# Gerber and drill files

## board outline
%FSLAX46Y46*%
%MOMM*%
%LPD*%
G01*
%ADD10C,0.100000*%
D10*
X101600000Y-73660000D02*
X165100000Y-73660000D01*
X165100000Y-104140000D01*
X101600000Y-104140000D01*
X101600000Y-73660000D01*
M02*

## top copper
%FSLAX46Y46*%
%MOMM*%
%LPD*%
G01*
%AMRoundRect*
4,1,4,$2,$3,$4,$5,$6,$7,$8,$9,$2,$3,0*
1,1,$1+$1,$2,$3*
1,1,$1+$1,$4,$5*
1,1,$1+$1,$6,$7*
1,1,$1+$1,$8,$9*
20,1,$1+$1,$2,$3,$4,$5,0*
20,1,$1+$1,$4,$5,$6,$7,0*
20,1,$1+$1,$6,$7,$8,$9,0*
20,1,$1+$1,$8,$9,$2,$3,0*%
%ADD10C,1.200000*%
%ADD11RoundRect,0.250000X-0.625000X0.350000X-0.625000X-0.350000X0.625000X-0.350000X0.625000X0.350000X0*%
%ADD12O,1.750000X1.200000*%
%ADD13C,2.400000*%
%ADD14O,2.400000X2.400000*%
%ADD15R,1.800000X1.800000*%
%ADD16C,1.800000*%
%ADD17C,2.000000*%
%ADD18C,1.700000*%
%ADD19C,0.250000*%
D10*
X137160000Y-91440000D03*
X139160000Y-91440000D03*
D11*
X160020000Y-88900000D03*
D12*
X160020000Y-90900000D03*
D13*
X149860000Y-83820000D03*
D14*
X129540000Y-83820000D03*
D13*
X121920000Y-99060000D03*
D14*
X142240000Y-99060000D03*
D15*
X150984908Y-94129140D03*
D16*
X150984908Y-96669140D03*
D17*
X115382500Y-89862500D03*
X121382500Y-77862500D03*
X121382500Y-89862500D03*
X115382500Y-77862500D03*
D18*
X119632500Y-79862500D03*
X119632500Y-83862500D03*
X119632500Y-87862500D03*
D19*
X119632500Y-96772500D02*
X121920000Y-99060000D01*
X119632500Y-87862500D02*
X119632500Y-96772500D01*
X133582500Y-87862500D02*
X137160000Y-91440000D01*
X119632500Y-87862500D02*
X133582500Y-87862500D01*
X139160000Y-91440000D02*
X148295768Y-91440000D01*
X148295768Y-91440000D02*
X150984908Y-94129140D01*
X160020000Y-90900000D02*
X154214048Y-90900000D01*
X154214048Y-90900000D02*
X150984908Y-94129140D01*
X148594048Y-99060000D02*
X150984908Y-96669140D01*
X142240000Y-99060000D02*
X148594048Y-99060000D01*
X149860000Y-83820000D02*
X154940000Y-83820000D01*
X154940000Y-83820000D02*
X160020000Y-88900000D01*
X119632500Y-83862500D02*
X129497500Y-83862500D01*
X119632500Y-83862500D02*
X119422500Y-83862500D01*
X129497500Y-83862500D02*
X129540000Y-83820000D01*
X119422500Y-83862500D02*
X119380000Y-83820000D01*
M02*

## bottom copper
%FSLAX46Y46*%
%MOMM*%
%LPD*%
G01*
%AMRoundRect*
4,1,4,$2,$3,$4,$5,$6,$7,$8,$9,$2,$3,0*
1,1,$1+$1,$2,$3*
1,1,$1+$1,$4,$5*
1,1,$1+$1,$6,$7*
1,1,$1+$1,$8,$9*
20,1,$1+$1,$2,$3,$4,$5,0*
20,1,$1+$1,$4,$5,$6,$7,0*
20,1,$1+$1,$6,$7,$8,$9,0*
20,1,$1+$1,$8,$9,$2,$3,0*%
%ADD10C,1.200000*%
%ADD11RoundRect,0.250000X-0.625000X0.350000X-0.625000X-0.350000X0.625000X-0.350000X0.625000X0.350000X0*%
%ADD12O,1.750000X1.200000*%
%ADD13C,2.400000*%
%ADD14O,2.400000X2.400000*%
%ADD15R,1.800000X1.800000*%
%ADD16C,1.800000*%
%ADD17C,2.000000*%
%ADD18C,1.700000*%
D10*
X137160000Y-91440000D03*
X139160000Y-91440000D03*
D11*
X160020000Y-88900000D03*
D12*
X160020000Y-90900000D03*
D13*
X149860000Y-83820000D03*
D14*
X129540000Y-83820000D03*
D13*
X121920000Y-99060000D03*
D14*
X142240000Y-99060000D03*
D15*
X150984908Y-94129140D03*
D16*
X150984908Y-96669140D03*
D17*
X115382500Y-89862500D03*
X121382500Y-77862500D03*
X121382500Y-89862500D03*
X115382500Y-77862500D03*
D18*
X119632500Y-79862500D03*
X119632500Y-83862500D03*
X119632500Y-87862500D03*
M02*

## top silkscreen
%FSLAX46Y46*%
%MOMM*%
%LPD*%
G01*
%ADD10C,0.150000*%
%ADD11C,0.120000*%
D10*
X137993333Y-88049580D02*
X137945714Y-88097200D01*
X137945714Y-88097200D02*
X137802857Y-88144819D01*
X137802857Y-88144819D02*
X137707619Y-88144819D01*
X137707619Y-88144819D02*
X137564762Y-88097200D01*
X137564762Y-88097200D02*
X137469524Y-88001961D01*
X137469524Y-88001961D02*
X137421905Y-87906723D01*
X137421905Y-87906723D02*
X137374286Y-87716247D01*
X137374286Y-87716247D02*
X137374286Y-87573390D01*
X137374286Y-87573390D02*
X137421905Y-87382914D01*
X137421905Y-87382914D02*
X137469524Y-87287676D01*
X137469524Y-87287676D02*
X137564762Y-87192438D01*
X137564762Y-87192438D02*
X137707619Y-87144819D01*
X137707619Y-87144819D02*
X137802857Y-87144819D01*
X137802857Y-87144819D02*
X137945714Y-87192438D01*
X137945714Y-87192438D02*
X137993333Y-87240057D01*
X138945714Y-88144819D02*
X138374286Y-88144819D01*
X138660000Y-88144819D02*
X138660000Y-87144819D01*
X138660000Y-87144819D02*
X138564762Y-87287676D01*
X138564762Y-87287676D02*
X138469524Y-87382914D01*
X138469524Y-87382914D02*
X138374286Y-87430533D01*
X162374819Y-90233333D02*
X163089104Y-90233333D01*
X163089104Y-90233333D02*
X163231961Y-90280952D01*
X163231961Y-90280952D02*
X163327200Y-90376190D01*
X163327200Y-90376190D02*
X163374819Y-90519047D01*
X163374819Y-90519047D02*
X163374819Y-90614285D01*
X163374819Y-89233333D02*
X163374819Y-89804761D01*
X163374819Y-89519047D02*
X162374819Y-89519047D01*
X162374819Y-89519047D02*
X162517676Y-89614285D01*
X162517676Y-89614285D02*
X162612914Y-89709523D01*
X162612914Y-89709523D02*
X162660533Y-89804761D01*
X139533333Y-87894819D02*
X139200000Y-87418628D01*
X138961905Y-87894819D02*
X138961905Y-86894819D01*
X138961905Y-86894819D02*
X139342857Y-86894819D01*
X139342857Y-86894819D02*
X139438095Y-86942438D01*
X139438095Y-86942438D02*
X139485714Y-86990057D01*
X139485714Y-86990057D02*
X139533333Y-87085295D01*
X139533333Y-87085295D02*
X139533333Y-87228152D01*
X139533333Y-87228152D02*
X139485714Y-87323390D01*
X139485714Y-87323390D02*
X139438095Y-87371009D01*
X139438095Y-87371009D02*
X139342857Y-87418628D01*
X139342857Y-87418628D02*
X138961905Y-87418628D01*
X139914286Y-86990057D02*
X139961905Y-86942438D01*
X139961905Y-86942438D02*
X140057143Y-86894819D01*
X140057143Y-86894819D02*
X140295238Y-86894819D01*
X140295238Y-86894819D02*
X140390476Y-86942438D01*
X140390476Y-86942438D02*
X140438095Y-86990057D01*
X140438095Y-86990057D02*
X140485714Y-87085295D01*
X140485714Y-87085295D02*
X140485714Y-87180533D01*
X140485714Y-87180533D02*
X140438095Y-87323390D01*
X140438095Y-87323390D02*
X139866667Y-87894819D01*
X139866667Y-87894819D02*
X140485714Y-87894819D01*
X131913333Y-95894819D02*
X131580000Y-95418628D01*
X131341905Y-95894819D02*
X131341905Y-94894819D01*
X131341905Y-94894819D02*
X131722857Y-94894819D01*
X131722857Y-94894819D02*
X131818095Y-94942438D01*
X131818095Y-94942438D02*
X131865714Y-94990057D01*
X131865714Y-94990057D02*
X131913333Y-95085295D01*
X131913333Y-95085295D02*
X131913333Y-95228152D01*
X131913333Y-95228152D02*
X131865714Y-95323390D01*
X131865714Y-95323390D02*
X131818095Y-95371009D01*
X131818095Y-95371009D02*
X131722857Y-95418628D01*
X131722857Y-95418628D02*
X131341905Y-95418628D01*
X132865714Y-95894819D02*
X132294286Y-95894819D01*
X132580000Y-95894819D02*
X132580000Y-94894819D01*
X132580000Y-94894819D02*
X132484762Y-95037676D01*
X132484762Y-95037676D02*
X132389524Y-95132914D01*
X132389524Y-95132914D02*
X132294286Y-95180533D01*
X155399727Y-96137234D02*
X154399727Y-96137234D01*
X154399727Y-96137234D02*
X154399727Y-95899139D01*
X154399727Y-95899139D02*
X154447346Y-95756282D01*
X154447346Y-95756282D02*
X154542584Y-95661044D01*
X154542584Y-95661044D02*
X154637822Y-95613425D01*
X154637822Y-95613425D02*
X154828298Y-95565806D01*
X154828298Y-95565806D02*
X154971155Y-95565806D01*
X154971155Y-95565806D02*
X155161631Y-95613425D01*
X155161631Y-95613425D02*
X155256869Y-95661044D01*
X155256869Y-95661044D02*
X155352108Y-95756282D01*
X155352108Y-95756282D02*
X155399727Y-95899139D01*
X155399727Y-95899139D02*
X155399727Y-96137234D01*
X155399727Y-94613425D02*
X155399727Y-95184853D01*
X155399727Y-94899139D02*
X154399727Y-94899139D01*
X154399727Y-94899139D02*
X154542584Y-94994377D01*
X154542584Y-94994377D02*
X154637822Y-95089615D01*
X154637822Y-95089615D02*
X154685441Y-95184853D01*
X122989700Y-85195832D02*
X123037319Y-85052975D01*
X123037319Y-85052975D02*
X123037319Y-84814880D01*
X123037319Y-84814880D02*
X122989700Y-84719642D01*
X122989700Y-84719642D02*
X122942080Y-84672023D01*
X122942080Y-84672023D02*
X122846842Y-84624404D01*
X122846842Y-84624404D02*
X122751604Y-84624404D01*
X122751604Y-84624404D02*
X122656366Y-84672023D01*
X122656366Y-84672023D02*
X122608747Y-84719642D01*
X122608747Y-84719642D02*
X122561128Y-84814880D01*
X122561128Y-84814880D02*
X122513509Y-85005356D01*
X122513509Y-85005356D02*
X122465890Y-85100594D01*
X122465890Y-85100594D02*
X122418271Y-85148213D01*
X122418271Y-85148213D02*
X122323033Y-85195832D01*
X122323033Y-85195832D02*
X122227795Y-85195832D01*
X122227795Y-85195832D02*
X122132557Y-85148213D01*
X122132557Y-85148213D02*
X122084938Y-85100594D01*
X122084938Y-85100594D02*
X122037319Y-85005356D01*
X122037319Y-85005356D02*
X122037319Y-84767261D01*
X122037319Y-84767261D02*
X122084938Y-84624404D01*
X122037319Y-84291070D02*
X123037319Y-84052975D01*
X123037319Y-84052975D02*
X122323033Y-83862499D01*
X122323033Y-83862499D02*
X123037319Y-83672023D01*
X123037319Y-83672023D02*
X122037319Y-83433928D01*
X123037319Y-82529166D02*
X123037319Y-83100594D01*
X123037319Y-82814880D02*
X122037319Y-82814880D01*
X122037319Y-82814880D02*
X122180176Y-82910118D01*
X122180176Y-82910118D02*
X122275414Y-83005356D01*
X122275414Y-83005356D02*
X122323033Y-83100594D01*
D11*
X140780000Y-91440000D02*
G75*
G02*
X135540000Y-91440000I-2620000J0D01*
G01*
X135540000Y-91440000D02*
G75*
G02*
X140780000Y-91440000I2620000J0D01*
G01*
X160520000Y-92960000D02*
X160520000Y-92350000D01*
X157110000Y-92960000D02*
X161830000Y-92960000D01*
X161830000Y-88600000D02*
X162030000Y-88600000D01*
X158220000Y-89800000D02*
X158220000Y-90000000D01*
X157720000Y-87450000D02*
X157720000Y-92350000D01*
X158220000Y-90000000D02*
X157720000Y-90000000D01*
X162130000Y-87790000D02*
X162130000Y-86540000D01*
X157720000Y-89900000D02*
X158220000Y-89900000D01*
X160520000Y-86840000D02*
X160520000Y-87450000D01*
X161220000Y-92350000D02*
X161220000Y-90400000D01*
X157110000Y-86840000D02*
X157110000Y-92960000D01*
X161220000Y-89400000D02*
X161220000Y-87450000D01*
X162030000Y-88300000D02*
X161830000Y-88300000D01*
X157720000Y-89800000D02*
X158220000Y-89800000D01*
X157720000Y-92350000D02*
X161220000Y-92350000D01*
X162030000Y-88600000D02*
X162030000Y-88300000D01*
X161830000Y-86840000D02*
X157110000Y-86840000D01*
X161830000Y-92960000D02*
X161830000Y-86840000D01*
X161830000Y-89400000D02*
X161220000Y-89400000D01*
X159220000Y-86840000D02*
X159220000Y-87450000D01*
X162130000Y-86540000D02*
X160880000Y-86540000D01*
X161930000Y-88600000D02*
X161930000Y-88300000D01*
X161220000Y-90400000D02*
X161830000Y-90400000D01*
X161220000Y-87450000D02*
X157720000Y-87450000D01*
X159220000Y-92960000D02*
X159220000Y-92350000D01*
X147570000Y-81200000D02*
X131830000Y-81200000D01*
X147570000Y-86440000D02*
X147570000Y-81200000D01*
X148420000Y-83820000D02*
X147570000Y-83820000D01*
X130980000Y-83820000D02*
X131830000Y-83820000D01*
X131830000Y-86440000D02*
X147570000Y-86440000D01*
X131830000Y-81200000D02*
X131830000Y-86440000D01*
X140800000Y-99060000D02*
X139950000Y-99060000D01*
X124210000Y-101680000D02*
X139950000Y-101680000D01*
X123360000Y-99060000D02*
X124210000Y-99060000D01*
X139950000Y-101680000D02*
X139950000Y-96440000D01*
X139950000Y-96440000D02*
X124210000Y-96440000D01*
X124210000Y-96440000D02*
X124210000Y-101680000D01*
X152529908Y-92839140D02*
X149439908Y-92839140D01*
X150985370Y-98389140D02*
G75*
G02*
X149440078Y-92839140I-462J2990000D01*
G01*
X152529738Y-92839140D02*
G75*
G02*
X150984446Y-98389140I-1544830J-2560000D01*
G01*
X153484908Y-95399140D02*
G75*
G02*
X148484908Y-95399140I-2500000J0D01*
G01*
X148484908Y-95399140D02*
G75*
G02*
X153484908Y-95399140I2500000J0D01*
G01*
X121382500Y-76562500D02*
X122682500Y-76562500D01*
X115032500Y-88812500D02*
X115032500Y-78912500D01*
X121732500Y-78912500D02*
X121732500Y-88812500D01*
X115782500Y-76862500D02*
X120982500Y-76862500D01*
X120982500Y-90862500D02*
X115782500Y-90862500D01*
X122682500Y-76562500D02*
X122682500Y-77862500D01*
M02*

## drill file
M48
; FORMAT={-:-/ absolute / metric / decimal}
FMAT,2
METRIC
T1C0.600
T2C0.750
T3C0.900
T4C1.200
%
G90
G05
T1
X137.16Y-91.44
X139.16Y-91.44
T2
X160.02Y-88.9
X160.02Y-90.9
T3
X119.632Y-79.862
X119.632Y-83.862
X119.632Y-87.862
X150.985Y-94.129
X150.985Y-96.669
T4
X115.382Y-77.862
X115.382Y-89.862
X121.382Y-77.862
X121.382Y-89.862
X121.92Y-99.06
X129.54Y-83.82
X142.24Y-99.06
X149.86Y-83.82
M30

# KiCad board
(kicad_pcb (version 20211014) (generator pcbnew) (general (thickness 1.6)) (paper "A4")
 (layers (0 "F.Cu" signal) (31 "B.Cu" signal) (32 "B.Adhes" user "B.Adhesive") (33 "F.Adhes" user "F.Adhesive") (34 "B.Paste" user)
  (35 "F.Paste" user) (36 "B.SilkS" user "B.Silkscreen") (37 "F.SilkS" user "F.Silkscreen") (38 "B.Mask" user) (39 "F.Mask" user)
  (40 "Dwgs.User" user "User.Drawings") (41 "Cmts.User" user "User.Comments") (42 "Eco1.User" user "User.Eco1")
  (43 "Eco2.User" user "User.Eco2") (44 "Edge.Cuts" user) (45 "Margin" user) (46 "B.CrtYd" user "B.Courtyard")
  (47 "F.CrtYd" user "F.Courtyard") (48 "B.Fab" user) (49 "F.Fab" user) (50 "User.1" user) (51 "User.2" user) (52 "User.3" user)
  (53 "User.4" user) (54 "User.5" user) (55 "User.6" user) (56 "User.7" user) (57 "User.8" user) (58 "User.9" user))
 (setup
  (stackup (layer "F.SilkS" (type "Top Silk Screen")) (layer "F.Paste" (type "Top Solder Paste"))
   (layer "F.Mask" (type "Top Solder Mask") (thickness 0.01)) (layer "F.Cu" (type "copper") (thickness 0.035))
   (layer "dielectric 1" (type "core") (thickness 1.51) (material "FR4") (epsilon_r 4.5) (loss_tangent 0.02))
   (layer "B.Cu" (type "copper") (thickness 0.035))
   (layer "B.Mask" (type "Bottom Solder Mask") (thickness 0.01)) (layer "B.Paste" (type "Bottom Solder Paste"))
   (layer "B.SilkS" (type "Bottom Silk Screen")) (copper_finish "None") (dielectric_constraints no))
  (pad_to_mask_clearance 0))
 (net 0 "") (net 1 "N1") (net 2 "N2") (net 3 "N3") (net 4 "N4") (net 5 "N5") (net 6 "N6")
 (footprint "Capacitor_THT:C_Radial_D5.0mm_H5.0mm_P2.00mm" (layer "F.Cu") (at 137.16 91.44)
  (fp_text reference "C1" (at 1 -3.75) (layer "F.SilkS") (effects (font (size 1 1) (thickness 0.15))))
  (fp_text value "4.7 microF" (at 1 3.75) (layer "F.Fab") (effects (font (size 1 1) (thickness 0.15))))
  (fp_circle (center 1 0) (end 3.62 0) (layer "F.SilkS") (width 0.12) (fill none))
  (pad "1" thru_hole circle (at 0 0) (size 1.2 1.2) (drill 0.6) (layers *.Cu *.Mask) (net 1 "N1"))
  (pad "2" thru_hole circle (at 2 0) (size 1.2 1.2) (drill 0.6) (layers *.Cu *.Mask) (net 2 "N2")))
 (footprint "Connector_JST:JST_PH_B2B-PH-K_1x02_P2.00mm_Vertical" (layer "F.Cu") (at 160.02 88.9 -90)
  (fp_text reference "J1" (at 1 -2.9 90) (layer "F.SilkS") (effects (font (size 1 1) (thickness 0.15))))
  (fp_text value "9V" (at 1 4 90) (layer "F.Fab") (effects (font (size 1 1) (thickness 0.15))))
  (fp_line (start 4.06 -0.5) (end 3.45 -0.5) (layer "F.SilkS") (width 0.12))
  (fp_line (start 4.06 2.91) (end 4.06 -1.81) (layer "F.SilkS") (width 0.12))
  (fp_line (start -0.3 -1.81) (end -0.3 -2.01) (layer "F.SilkS") (width 0.12))
  (fp_line (start 0.9 1.8) (end 1.1 1.8) (layer "F.SilkS") (width 0.12))
  (fp_line (start -1.45 2.3) (end 3.45 2.3) (layer "F.SilkS") (width 0.12))
  (fp_line (start 1.1 1.8) (end 1.1 2.3) (layer "F.SilkS") (width 0.12))
  (fp_line (start -1.11 -2.11) (end -2.36 -2.11) (layer "F.SilkS") (width 0.12))
  (fp_line (start 1 2.3) (end 1 1.8) (layer "F.SilkS") (width 0.12))
  (fp_line (start -2.06 -0.5) (end -1.45 -0.5) (layer "F.SilkS") (width 0.12))
  (fp_line (start 3.45 -1.2) (end 1.5 -1.2) (layer "F.SilkS") (width 0.12))
  (fp_line (start -2.06 2.91) (end 4.06 2.91) (layer "F.SilkS") (width 0.12))
  (fp_line (start 0.5 -1.2) (end -1.45 -1.2) (layer "F.SilkS") (width 0.12))
  (fp_line (start -0.6 -2.01) (end -0.6 -1.81) (layer "F.SilkS") (width 0.12))
  (fp_line (start 0.9 2.3) (end 0.9 1.8) (layer "F.SilkS") (width 0.12))
  (fp_line (start 3.45 2.3) (end 3.45 -1.2) (layer "F.SilkS") (width 0.12))
  (fp_line (start -0.3 -2.01) (end -0.6 -2.01) (layer "F.SilkS") (width 0.12))
  (fp_line (start -2.06 -1.81) (end -2.06 2.91) (layer "F.SilkS") (width 0.12))
  (fp_line (start 4.06 -1.81) (end -2.06 -1.81) (layer "F.SilkS") (width 0.12))
  (fp_line (start 0.5 -1.81) (end 0.5 -1.2) (layer "F.SilkS") (width 0.12))
  (fp_line (start -2.06 0.8) (end -1.45 0.8) (layer "F.SilkS") (width 0.12))
  (fp_line (start -2.36 -2.11) (end -2.36 -0.86) (layer "F.SilkS") (width 0.12))
  (fp_line (start -0.3 -1.91) (end -0.6 -1.91) (layer "F.SilkS") (width 0.12))
  (fp_line (start 1.5 -1.2) (end 1.5 -1.81) (layer "F.SilkS") (width 0.12))
  (fp_line (start -1.45 -1.2) (end -1.45 2.3) (layer "F.SilkS") (width 0.12))
  (fp_line (start 4.06 0.8) (end 3.45 0.8) (layer "F.SilkS") (width 0.12))
  (pad "1" thru_hole roundrect (at 0 0 270) (size 1.2 1.75) (drill 0.75) (layers *.Cu *.Mask) (roundrect_rratio 0.2083333333) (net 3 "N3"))
  (pad "2" thru_hole oval (at 2 0 270) (size 1.2 1.75) (drill 0.75) (layers *.Cu *.Mask) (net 2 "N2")))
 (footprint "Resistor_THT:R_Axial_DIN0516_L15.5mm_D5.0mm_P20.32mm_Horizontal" (layer "F.Cu") (at 149.86 83.82 180)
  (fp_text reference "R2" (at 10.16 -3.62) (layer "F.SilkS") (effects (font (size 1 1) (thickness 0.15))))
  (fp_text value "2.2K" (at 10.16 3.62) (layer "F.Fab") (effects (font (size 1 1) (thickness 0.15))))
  (fp_line (start 2.29 2.62) (end 18.03 2.62) (layer "F.SilkS") (width 0.12))
  (fp_line (start 2.29 -2.62) (end 2.29 2.62) (layer "F.SilkS") (width 0.12))
  (fp_line (start 1.44 0) (end 2.29 0) (layer "F.SilkS") (width 0.12))
  (fp_line (start 18.88 0) (end 18.03 0) (layer "F.SilkS") (width 0.12))
  (fp_line (start 18.03 -2.62) (end 2.29 -2.62) (layer "F.SilkS") (width 0.12))
  (fp_line (start 18.03 2.62) (end 18.03 -2.62) (layer "F.SilkS") (width 0.12))
  (pad "1" thru_hole circle (at 0 0 180) (size 2.4 2.4) (drill 1.2) (layers *.Cu *.Mask) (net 3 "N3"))
  (pad "2" thru_hole oval (at 20.32 0 180) (size 2.4 2.4) (drill 1.2) (layers *.Cu *.Mask) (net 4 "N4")))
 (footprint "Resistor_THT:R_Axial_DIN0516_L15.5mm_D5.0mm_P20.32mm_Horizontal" (layer "F.Cu") (at 121.92 99.06)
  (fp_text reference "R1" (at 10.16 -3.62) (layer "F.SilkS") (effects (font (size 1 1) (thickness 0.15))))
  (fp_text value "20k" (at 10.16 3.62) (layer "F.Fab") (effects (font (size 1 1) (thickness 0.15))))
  (fp_line (start 18.88 0) (end 18.03 0) (layer "F.SilkS") (width 0.12))
  (fp_line (start 2.29 2.62) (end 18.03 2.62) (layer "F.SilkS") (width 0.12))
  (fp_line (start 1.44 0) (end 2.29 0) (layer "F.SilkS") (width 0.12))
  (fp_line (start 18.03 2.62) (end 18.03 -2.62) (layer "F.SilkS") (width 0.12))
  (fp_line (start 18.03 -2.62) (end 2.29 -2.62) (layer "F.SilkS") (width 0.12))
  (fp_line (start 2.29 -2.62) (end 2.29 2.62) (layer "F.SilkS") (width 0.12))
  (pad "1" thru_hole circle (at 0 0) (size 2.4 2.4) (drill 1.2) (layers *.Cu *.Mask) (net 1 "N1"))
  (pad "2" thru_hole oval (at 20.32 0) (size 2.4 2.4) (drill 1.2) (layers *.Cu *.Mask) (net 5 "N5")))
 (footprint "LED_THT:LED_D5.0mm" (layer "F.Cu") (at 150.984908 94.12914 -90)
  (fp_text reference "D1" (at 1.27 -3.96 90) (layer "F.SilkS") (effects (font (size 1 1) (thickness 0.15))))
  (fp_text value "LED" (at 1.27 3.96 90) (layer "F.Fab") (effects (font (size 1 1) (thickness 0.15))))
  (fp_line (start -1.29 -1.545) (end -1.29 1.545) (layer "F.SilkS") (width 0.12))
  (fp_arc (start 4.26 -0.000462) (mid 2.072002 2.880433) (end -1.29 1.54483) (layer "F.SilkS") (width 0.12))
  (fp_arc (start -1.29 -1.54483) (mid 2.072002 -2.880433) (end 4.26 0.000462) (layer "F.SilkS") (width 0.12))
  (fp_circle (center 1.27 0) (end 3.77 0) (layer "F.SilkS") (width 0.12) (fill none))
  (pad "1" thru_hole rect (at 0 0 270) (size 1.8 1.8) (drill 0.9) (layers *.Cu *.Mask) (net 2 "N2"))
  (pad "2" thru_hole circle (at 2.54 0 270) (size 1.8 1.8) (drill 0.9) (layers *.Cu *.Mask) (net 5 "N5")))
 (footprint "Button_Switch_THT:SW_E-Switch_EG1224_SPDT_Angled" (layer "F.Cu") (at 119.6325 79.8625 -90)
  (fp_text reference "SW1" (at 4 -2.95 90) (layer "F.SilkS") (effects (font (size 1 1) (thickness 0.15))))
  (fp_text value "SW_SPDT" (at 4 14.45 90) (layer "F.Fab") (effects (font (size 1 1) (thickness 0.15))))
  (fp_line (start -3.3 -1.75) (end -3.3 -3.05) (layer "F.SilkS") (width 0.12))
  (fp_line (start 8.95 4.6) (end -0.95 4.6) (layer "F.SilkS") (width 0.12))
  (fp_line (start -0.95 -2.1) (end 8.95 -2.1) (layer "F.SilkS") (width 0.12))
  (fp_line (start -3 3.85) (end -3 -1.35) (layer "F.SilkS") (width 0.12))
  (fp_line (start 11 -1.35) (end 11 3.85) (layer "F.SilkS") (width 0.12))
  (fp_line (start -3.3 -3.05) (end -2 -3.05) (layer "F.SilkS") (width 0.12))
  (pad "" thru_hole circle (at 10 4.25 270) (size 2 2) (drill 1.2) (layers *.Cu *.Mask))
  (pad "" thru_hole circle (at -2 -1.75 270) (size 2 2) (drill 1.2) (layers *.Cu *.Mask))
  (pad "" thru_hole circle (at 10 -1.75 270) (size 2 2) (drill 1.2) (layers *.Cu *.Mask))
  (pad "" thru_hole circle (at -2 4.25 270) (size 2 2) (drill 1.2) (layers *.Cu *.Mask))
  (pad "1" thru_hole circle (at 0 0 270) (size 1.7 1.7) (drill 0.9) (layers *.Cu *.Mask) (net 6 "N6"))
  (pad "2" thru_hole circle (at 4 0 270) (size 1.7 1.7) (drill 0.9) (layers *.Cu *.Mask) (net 4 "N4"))
  (pad "3" thru_hole circle (at 8 0 270) (size 1.7 1.7) (drill 0.9) (layers *.Cu *.Mask) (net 1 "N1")))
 (gr_rect (start 101.6 73.66) (end 165.1 104.14) (layer "Edge.Cuts") (width 0.1) (fill none))
 (segment (start 119.6325 96.7725) (end 121.92 99.06) (width 0.25) (layer "F.Cu") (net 1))
 (segment (start 119.6325 87.8625) (end 119.6325 96.7725) (width 0.25) (layer "F.Cu") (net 1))
 (segment (start 133.5825 87.8625) (end 137.16 91.44) (width 0.25) (layer "F.Cu") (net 1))
 (segment (start 119.6325 87.8625) (end 133.5825 87.8625) (width 0.25) (layer "F.Cu") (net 1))
 (segment (start 139.16 91.44) (end 148.295768 91.44) (width 0.25) (layer "F.Cu") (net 2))
 (segment (start 148.295768 91.44) (end 150.984908 94.12914) (width 0.25) (layer "F.Cu") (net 2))
 (segment (start 160.02 90.9) (end 154.214048 90.9) (width 0.25) (layer "F.Cu") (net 2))
 (segment (start 154.214048 90.9) (end 150.984908 94.12914) (width 0.25) (layer "F.Cu") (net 2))
 (segment (start 148.594048 99.06) (end 150.984908 96.66914) (width 0.25) (layer "F.Cu") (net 5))
 (segment (start 142.24 99.06) (end 148.594048 99.06) (width 0.25) (layer "F.Cu") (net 5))
 (segment (start 149.86 83.82) (end 154.94 83.82) (width 0.25) (layer "F.Cu") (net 3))
 (segment (start 154.94 83.82) (end 160.02 88.9) (width 0.25) (layer "F.Cu") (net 3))
 (segment (start 119.6325 83.8625) (end 129.4975 83.8625) (width 0.25) (layer "F.Cu") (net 4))
 (segment (start 119.6325 83.8625) (end 119.4225 83.8625) (width 0.25) (layer "F.Cu") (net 4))
 (segment (start 129.4975 83.8625) (end 129.54 83.82) (width 0.25) (layer "F.Cu") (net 4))
 (segment (start 119.4225 83.8625) (end 119.38 83.82) (width 0.25) (layer "F.Cu") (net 4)))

